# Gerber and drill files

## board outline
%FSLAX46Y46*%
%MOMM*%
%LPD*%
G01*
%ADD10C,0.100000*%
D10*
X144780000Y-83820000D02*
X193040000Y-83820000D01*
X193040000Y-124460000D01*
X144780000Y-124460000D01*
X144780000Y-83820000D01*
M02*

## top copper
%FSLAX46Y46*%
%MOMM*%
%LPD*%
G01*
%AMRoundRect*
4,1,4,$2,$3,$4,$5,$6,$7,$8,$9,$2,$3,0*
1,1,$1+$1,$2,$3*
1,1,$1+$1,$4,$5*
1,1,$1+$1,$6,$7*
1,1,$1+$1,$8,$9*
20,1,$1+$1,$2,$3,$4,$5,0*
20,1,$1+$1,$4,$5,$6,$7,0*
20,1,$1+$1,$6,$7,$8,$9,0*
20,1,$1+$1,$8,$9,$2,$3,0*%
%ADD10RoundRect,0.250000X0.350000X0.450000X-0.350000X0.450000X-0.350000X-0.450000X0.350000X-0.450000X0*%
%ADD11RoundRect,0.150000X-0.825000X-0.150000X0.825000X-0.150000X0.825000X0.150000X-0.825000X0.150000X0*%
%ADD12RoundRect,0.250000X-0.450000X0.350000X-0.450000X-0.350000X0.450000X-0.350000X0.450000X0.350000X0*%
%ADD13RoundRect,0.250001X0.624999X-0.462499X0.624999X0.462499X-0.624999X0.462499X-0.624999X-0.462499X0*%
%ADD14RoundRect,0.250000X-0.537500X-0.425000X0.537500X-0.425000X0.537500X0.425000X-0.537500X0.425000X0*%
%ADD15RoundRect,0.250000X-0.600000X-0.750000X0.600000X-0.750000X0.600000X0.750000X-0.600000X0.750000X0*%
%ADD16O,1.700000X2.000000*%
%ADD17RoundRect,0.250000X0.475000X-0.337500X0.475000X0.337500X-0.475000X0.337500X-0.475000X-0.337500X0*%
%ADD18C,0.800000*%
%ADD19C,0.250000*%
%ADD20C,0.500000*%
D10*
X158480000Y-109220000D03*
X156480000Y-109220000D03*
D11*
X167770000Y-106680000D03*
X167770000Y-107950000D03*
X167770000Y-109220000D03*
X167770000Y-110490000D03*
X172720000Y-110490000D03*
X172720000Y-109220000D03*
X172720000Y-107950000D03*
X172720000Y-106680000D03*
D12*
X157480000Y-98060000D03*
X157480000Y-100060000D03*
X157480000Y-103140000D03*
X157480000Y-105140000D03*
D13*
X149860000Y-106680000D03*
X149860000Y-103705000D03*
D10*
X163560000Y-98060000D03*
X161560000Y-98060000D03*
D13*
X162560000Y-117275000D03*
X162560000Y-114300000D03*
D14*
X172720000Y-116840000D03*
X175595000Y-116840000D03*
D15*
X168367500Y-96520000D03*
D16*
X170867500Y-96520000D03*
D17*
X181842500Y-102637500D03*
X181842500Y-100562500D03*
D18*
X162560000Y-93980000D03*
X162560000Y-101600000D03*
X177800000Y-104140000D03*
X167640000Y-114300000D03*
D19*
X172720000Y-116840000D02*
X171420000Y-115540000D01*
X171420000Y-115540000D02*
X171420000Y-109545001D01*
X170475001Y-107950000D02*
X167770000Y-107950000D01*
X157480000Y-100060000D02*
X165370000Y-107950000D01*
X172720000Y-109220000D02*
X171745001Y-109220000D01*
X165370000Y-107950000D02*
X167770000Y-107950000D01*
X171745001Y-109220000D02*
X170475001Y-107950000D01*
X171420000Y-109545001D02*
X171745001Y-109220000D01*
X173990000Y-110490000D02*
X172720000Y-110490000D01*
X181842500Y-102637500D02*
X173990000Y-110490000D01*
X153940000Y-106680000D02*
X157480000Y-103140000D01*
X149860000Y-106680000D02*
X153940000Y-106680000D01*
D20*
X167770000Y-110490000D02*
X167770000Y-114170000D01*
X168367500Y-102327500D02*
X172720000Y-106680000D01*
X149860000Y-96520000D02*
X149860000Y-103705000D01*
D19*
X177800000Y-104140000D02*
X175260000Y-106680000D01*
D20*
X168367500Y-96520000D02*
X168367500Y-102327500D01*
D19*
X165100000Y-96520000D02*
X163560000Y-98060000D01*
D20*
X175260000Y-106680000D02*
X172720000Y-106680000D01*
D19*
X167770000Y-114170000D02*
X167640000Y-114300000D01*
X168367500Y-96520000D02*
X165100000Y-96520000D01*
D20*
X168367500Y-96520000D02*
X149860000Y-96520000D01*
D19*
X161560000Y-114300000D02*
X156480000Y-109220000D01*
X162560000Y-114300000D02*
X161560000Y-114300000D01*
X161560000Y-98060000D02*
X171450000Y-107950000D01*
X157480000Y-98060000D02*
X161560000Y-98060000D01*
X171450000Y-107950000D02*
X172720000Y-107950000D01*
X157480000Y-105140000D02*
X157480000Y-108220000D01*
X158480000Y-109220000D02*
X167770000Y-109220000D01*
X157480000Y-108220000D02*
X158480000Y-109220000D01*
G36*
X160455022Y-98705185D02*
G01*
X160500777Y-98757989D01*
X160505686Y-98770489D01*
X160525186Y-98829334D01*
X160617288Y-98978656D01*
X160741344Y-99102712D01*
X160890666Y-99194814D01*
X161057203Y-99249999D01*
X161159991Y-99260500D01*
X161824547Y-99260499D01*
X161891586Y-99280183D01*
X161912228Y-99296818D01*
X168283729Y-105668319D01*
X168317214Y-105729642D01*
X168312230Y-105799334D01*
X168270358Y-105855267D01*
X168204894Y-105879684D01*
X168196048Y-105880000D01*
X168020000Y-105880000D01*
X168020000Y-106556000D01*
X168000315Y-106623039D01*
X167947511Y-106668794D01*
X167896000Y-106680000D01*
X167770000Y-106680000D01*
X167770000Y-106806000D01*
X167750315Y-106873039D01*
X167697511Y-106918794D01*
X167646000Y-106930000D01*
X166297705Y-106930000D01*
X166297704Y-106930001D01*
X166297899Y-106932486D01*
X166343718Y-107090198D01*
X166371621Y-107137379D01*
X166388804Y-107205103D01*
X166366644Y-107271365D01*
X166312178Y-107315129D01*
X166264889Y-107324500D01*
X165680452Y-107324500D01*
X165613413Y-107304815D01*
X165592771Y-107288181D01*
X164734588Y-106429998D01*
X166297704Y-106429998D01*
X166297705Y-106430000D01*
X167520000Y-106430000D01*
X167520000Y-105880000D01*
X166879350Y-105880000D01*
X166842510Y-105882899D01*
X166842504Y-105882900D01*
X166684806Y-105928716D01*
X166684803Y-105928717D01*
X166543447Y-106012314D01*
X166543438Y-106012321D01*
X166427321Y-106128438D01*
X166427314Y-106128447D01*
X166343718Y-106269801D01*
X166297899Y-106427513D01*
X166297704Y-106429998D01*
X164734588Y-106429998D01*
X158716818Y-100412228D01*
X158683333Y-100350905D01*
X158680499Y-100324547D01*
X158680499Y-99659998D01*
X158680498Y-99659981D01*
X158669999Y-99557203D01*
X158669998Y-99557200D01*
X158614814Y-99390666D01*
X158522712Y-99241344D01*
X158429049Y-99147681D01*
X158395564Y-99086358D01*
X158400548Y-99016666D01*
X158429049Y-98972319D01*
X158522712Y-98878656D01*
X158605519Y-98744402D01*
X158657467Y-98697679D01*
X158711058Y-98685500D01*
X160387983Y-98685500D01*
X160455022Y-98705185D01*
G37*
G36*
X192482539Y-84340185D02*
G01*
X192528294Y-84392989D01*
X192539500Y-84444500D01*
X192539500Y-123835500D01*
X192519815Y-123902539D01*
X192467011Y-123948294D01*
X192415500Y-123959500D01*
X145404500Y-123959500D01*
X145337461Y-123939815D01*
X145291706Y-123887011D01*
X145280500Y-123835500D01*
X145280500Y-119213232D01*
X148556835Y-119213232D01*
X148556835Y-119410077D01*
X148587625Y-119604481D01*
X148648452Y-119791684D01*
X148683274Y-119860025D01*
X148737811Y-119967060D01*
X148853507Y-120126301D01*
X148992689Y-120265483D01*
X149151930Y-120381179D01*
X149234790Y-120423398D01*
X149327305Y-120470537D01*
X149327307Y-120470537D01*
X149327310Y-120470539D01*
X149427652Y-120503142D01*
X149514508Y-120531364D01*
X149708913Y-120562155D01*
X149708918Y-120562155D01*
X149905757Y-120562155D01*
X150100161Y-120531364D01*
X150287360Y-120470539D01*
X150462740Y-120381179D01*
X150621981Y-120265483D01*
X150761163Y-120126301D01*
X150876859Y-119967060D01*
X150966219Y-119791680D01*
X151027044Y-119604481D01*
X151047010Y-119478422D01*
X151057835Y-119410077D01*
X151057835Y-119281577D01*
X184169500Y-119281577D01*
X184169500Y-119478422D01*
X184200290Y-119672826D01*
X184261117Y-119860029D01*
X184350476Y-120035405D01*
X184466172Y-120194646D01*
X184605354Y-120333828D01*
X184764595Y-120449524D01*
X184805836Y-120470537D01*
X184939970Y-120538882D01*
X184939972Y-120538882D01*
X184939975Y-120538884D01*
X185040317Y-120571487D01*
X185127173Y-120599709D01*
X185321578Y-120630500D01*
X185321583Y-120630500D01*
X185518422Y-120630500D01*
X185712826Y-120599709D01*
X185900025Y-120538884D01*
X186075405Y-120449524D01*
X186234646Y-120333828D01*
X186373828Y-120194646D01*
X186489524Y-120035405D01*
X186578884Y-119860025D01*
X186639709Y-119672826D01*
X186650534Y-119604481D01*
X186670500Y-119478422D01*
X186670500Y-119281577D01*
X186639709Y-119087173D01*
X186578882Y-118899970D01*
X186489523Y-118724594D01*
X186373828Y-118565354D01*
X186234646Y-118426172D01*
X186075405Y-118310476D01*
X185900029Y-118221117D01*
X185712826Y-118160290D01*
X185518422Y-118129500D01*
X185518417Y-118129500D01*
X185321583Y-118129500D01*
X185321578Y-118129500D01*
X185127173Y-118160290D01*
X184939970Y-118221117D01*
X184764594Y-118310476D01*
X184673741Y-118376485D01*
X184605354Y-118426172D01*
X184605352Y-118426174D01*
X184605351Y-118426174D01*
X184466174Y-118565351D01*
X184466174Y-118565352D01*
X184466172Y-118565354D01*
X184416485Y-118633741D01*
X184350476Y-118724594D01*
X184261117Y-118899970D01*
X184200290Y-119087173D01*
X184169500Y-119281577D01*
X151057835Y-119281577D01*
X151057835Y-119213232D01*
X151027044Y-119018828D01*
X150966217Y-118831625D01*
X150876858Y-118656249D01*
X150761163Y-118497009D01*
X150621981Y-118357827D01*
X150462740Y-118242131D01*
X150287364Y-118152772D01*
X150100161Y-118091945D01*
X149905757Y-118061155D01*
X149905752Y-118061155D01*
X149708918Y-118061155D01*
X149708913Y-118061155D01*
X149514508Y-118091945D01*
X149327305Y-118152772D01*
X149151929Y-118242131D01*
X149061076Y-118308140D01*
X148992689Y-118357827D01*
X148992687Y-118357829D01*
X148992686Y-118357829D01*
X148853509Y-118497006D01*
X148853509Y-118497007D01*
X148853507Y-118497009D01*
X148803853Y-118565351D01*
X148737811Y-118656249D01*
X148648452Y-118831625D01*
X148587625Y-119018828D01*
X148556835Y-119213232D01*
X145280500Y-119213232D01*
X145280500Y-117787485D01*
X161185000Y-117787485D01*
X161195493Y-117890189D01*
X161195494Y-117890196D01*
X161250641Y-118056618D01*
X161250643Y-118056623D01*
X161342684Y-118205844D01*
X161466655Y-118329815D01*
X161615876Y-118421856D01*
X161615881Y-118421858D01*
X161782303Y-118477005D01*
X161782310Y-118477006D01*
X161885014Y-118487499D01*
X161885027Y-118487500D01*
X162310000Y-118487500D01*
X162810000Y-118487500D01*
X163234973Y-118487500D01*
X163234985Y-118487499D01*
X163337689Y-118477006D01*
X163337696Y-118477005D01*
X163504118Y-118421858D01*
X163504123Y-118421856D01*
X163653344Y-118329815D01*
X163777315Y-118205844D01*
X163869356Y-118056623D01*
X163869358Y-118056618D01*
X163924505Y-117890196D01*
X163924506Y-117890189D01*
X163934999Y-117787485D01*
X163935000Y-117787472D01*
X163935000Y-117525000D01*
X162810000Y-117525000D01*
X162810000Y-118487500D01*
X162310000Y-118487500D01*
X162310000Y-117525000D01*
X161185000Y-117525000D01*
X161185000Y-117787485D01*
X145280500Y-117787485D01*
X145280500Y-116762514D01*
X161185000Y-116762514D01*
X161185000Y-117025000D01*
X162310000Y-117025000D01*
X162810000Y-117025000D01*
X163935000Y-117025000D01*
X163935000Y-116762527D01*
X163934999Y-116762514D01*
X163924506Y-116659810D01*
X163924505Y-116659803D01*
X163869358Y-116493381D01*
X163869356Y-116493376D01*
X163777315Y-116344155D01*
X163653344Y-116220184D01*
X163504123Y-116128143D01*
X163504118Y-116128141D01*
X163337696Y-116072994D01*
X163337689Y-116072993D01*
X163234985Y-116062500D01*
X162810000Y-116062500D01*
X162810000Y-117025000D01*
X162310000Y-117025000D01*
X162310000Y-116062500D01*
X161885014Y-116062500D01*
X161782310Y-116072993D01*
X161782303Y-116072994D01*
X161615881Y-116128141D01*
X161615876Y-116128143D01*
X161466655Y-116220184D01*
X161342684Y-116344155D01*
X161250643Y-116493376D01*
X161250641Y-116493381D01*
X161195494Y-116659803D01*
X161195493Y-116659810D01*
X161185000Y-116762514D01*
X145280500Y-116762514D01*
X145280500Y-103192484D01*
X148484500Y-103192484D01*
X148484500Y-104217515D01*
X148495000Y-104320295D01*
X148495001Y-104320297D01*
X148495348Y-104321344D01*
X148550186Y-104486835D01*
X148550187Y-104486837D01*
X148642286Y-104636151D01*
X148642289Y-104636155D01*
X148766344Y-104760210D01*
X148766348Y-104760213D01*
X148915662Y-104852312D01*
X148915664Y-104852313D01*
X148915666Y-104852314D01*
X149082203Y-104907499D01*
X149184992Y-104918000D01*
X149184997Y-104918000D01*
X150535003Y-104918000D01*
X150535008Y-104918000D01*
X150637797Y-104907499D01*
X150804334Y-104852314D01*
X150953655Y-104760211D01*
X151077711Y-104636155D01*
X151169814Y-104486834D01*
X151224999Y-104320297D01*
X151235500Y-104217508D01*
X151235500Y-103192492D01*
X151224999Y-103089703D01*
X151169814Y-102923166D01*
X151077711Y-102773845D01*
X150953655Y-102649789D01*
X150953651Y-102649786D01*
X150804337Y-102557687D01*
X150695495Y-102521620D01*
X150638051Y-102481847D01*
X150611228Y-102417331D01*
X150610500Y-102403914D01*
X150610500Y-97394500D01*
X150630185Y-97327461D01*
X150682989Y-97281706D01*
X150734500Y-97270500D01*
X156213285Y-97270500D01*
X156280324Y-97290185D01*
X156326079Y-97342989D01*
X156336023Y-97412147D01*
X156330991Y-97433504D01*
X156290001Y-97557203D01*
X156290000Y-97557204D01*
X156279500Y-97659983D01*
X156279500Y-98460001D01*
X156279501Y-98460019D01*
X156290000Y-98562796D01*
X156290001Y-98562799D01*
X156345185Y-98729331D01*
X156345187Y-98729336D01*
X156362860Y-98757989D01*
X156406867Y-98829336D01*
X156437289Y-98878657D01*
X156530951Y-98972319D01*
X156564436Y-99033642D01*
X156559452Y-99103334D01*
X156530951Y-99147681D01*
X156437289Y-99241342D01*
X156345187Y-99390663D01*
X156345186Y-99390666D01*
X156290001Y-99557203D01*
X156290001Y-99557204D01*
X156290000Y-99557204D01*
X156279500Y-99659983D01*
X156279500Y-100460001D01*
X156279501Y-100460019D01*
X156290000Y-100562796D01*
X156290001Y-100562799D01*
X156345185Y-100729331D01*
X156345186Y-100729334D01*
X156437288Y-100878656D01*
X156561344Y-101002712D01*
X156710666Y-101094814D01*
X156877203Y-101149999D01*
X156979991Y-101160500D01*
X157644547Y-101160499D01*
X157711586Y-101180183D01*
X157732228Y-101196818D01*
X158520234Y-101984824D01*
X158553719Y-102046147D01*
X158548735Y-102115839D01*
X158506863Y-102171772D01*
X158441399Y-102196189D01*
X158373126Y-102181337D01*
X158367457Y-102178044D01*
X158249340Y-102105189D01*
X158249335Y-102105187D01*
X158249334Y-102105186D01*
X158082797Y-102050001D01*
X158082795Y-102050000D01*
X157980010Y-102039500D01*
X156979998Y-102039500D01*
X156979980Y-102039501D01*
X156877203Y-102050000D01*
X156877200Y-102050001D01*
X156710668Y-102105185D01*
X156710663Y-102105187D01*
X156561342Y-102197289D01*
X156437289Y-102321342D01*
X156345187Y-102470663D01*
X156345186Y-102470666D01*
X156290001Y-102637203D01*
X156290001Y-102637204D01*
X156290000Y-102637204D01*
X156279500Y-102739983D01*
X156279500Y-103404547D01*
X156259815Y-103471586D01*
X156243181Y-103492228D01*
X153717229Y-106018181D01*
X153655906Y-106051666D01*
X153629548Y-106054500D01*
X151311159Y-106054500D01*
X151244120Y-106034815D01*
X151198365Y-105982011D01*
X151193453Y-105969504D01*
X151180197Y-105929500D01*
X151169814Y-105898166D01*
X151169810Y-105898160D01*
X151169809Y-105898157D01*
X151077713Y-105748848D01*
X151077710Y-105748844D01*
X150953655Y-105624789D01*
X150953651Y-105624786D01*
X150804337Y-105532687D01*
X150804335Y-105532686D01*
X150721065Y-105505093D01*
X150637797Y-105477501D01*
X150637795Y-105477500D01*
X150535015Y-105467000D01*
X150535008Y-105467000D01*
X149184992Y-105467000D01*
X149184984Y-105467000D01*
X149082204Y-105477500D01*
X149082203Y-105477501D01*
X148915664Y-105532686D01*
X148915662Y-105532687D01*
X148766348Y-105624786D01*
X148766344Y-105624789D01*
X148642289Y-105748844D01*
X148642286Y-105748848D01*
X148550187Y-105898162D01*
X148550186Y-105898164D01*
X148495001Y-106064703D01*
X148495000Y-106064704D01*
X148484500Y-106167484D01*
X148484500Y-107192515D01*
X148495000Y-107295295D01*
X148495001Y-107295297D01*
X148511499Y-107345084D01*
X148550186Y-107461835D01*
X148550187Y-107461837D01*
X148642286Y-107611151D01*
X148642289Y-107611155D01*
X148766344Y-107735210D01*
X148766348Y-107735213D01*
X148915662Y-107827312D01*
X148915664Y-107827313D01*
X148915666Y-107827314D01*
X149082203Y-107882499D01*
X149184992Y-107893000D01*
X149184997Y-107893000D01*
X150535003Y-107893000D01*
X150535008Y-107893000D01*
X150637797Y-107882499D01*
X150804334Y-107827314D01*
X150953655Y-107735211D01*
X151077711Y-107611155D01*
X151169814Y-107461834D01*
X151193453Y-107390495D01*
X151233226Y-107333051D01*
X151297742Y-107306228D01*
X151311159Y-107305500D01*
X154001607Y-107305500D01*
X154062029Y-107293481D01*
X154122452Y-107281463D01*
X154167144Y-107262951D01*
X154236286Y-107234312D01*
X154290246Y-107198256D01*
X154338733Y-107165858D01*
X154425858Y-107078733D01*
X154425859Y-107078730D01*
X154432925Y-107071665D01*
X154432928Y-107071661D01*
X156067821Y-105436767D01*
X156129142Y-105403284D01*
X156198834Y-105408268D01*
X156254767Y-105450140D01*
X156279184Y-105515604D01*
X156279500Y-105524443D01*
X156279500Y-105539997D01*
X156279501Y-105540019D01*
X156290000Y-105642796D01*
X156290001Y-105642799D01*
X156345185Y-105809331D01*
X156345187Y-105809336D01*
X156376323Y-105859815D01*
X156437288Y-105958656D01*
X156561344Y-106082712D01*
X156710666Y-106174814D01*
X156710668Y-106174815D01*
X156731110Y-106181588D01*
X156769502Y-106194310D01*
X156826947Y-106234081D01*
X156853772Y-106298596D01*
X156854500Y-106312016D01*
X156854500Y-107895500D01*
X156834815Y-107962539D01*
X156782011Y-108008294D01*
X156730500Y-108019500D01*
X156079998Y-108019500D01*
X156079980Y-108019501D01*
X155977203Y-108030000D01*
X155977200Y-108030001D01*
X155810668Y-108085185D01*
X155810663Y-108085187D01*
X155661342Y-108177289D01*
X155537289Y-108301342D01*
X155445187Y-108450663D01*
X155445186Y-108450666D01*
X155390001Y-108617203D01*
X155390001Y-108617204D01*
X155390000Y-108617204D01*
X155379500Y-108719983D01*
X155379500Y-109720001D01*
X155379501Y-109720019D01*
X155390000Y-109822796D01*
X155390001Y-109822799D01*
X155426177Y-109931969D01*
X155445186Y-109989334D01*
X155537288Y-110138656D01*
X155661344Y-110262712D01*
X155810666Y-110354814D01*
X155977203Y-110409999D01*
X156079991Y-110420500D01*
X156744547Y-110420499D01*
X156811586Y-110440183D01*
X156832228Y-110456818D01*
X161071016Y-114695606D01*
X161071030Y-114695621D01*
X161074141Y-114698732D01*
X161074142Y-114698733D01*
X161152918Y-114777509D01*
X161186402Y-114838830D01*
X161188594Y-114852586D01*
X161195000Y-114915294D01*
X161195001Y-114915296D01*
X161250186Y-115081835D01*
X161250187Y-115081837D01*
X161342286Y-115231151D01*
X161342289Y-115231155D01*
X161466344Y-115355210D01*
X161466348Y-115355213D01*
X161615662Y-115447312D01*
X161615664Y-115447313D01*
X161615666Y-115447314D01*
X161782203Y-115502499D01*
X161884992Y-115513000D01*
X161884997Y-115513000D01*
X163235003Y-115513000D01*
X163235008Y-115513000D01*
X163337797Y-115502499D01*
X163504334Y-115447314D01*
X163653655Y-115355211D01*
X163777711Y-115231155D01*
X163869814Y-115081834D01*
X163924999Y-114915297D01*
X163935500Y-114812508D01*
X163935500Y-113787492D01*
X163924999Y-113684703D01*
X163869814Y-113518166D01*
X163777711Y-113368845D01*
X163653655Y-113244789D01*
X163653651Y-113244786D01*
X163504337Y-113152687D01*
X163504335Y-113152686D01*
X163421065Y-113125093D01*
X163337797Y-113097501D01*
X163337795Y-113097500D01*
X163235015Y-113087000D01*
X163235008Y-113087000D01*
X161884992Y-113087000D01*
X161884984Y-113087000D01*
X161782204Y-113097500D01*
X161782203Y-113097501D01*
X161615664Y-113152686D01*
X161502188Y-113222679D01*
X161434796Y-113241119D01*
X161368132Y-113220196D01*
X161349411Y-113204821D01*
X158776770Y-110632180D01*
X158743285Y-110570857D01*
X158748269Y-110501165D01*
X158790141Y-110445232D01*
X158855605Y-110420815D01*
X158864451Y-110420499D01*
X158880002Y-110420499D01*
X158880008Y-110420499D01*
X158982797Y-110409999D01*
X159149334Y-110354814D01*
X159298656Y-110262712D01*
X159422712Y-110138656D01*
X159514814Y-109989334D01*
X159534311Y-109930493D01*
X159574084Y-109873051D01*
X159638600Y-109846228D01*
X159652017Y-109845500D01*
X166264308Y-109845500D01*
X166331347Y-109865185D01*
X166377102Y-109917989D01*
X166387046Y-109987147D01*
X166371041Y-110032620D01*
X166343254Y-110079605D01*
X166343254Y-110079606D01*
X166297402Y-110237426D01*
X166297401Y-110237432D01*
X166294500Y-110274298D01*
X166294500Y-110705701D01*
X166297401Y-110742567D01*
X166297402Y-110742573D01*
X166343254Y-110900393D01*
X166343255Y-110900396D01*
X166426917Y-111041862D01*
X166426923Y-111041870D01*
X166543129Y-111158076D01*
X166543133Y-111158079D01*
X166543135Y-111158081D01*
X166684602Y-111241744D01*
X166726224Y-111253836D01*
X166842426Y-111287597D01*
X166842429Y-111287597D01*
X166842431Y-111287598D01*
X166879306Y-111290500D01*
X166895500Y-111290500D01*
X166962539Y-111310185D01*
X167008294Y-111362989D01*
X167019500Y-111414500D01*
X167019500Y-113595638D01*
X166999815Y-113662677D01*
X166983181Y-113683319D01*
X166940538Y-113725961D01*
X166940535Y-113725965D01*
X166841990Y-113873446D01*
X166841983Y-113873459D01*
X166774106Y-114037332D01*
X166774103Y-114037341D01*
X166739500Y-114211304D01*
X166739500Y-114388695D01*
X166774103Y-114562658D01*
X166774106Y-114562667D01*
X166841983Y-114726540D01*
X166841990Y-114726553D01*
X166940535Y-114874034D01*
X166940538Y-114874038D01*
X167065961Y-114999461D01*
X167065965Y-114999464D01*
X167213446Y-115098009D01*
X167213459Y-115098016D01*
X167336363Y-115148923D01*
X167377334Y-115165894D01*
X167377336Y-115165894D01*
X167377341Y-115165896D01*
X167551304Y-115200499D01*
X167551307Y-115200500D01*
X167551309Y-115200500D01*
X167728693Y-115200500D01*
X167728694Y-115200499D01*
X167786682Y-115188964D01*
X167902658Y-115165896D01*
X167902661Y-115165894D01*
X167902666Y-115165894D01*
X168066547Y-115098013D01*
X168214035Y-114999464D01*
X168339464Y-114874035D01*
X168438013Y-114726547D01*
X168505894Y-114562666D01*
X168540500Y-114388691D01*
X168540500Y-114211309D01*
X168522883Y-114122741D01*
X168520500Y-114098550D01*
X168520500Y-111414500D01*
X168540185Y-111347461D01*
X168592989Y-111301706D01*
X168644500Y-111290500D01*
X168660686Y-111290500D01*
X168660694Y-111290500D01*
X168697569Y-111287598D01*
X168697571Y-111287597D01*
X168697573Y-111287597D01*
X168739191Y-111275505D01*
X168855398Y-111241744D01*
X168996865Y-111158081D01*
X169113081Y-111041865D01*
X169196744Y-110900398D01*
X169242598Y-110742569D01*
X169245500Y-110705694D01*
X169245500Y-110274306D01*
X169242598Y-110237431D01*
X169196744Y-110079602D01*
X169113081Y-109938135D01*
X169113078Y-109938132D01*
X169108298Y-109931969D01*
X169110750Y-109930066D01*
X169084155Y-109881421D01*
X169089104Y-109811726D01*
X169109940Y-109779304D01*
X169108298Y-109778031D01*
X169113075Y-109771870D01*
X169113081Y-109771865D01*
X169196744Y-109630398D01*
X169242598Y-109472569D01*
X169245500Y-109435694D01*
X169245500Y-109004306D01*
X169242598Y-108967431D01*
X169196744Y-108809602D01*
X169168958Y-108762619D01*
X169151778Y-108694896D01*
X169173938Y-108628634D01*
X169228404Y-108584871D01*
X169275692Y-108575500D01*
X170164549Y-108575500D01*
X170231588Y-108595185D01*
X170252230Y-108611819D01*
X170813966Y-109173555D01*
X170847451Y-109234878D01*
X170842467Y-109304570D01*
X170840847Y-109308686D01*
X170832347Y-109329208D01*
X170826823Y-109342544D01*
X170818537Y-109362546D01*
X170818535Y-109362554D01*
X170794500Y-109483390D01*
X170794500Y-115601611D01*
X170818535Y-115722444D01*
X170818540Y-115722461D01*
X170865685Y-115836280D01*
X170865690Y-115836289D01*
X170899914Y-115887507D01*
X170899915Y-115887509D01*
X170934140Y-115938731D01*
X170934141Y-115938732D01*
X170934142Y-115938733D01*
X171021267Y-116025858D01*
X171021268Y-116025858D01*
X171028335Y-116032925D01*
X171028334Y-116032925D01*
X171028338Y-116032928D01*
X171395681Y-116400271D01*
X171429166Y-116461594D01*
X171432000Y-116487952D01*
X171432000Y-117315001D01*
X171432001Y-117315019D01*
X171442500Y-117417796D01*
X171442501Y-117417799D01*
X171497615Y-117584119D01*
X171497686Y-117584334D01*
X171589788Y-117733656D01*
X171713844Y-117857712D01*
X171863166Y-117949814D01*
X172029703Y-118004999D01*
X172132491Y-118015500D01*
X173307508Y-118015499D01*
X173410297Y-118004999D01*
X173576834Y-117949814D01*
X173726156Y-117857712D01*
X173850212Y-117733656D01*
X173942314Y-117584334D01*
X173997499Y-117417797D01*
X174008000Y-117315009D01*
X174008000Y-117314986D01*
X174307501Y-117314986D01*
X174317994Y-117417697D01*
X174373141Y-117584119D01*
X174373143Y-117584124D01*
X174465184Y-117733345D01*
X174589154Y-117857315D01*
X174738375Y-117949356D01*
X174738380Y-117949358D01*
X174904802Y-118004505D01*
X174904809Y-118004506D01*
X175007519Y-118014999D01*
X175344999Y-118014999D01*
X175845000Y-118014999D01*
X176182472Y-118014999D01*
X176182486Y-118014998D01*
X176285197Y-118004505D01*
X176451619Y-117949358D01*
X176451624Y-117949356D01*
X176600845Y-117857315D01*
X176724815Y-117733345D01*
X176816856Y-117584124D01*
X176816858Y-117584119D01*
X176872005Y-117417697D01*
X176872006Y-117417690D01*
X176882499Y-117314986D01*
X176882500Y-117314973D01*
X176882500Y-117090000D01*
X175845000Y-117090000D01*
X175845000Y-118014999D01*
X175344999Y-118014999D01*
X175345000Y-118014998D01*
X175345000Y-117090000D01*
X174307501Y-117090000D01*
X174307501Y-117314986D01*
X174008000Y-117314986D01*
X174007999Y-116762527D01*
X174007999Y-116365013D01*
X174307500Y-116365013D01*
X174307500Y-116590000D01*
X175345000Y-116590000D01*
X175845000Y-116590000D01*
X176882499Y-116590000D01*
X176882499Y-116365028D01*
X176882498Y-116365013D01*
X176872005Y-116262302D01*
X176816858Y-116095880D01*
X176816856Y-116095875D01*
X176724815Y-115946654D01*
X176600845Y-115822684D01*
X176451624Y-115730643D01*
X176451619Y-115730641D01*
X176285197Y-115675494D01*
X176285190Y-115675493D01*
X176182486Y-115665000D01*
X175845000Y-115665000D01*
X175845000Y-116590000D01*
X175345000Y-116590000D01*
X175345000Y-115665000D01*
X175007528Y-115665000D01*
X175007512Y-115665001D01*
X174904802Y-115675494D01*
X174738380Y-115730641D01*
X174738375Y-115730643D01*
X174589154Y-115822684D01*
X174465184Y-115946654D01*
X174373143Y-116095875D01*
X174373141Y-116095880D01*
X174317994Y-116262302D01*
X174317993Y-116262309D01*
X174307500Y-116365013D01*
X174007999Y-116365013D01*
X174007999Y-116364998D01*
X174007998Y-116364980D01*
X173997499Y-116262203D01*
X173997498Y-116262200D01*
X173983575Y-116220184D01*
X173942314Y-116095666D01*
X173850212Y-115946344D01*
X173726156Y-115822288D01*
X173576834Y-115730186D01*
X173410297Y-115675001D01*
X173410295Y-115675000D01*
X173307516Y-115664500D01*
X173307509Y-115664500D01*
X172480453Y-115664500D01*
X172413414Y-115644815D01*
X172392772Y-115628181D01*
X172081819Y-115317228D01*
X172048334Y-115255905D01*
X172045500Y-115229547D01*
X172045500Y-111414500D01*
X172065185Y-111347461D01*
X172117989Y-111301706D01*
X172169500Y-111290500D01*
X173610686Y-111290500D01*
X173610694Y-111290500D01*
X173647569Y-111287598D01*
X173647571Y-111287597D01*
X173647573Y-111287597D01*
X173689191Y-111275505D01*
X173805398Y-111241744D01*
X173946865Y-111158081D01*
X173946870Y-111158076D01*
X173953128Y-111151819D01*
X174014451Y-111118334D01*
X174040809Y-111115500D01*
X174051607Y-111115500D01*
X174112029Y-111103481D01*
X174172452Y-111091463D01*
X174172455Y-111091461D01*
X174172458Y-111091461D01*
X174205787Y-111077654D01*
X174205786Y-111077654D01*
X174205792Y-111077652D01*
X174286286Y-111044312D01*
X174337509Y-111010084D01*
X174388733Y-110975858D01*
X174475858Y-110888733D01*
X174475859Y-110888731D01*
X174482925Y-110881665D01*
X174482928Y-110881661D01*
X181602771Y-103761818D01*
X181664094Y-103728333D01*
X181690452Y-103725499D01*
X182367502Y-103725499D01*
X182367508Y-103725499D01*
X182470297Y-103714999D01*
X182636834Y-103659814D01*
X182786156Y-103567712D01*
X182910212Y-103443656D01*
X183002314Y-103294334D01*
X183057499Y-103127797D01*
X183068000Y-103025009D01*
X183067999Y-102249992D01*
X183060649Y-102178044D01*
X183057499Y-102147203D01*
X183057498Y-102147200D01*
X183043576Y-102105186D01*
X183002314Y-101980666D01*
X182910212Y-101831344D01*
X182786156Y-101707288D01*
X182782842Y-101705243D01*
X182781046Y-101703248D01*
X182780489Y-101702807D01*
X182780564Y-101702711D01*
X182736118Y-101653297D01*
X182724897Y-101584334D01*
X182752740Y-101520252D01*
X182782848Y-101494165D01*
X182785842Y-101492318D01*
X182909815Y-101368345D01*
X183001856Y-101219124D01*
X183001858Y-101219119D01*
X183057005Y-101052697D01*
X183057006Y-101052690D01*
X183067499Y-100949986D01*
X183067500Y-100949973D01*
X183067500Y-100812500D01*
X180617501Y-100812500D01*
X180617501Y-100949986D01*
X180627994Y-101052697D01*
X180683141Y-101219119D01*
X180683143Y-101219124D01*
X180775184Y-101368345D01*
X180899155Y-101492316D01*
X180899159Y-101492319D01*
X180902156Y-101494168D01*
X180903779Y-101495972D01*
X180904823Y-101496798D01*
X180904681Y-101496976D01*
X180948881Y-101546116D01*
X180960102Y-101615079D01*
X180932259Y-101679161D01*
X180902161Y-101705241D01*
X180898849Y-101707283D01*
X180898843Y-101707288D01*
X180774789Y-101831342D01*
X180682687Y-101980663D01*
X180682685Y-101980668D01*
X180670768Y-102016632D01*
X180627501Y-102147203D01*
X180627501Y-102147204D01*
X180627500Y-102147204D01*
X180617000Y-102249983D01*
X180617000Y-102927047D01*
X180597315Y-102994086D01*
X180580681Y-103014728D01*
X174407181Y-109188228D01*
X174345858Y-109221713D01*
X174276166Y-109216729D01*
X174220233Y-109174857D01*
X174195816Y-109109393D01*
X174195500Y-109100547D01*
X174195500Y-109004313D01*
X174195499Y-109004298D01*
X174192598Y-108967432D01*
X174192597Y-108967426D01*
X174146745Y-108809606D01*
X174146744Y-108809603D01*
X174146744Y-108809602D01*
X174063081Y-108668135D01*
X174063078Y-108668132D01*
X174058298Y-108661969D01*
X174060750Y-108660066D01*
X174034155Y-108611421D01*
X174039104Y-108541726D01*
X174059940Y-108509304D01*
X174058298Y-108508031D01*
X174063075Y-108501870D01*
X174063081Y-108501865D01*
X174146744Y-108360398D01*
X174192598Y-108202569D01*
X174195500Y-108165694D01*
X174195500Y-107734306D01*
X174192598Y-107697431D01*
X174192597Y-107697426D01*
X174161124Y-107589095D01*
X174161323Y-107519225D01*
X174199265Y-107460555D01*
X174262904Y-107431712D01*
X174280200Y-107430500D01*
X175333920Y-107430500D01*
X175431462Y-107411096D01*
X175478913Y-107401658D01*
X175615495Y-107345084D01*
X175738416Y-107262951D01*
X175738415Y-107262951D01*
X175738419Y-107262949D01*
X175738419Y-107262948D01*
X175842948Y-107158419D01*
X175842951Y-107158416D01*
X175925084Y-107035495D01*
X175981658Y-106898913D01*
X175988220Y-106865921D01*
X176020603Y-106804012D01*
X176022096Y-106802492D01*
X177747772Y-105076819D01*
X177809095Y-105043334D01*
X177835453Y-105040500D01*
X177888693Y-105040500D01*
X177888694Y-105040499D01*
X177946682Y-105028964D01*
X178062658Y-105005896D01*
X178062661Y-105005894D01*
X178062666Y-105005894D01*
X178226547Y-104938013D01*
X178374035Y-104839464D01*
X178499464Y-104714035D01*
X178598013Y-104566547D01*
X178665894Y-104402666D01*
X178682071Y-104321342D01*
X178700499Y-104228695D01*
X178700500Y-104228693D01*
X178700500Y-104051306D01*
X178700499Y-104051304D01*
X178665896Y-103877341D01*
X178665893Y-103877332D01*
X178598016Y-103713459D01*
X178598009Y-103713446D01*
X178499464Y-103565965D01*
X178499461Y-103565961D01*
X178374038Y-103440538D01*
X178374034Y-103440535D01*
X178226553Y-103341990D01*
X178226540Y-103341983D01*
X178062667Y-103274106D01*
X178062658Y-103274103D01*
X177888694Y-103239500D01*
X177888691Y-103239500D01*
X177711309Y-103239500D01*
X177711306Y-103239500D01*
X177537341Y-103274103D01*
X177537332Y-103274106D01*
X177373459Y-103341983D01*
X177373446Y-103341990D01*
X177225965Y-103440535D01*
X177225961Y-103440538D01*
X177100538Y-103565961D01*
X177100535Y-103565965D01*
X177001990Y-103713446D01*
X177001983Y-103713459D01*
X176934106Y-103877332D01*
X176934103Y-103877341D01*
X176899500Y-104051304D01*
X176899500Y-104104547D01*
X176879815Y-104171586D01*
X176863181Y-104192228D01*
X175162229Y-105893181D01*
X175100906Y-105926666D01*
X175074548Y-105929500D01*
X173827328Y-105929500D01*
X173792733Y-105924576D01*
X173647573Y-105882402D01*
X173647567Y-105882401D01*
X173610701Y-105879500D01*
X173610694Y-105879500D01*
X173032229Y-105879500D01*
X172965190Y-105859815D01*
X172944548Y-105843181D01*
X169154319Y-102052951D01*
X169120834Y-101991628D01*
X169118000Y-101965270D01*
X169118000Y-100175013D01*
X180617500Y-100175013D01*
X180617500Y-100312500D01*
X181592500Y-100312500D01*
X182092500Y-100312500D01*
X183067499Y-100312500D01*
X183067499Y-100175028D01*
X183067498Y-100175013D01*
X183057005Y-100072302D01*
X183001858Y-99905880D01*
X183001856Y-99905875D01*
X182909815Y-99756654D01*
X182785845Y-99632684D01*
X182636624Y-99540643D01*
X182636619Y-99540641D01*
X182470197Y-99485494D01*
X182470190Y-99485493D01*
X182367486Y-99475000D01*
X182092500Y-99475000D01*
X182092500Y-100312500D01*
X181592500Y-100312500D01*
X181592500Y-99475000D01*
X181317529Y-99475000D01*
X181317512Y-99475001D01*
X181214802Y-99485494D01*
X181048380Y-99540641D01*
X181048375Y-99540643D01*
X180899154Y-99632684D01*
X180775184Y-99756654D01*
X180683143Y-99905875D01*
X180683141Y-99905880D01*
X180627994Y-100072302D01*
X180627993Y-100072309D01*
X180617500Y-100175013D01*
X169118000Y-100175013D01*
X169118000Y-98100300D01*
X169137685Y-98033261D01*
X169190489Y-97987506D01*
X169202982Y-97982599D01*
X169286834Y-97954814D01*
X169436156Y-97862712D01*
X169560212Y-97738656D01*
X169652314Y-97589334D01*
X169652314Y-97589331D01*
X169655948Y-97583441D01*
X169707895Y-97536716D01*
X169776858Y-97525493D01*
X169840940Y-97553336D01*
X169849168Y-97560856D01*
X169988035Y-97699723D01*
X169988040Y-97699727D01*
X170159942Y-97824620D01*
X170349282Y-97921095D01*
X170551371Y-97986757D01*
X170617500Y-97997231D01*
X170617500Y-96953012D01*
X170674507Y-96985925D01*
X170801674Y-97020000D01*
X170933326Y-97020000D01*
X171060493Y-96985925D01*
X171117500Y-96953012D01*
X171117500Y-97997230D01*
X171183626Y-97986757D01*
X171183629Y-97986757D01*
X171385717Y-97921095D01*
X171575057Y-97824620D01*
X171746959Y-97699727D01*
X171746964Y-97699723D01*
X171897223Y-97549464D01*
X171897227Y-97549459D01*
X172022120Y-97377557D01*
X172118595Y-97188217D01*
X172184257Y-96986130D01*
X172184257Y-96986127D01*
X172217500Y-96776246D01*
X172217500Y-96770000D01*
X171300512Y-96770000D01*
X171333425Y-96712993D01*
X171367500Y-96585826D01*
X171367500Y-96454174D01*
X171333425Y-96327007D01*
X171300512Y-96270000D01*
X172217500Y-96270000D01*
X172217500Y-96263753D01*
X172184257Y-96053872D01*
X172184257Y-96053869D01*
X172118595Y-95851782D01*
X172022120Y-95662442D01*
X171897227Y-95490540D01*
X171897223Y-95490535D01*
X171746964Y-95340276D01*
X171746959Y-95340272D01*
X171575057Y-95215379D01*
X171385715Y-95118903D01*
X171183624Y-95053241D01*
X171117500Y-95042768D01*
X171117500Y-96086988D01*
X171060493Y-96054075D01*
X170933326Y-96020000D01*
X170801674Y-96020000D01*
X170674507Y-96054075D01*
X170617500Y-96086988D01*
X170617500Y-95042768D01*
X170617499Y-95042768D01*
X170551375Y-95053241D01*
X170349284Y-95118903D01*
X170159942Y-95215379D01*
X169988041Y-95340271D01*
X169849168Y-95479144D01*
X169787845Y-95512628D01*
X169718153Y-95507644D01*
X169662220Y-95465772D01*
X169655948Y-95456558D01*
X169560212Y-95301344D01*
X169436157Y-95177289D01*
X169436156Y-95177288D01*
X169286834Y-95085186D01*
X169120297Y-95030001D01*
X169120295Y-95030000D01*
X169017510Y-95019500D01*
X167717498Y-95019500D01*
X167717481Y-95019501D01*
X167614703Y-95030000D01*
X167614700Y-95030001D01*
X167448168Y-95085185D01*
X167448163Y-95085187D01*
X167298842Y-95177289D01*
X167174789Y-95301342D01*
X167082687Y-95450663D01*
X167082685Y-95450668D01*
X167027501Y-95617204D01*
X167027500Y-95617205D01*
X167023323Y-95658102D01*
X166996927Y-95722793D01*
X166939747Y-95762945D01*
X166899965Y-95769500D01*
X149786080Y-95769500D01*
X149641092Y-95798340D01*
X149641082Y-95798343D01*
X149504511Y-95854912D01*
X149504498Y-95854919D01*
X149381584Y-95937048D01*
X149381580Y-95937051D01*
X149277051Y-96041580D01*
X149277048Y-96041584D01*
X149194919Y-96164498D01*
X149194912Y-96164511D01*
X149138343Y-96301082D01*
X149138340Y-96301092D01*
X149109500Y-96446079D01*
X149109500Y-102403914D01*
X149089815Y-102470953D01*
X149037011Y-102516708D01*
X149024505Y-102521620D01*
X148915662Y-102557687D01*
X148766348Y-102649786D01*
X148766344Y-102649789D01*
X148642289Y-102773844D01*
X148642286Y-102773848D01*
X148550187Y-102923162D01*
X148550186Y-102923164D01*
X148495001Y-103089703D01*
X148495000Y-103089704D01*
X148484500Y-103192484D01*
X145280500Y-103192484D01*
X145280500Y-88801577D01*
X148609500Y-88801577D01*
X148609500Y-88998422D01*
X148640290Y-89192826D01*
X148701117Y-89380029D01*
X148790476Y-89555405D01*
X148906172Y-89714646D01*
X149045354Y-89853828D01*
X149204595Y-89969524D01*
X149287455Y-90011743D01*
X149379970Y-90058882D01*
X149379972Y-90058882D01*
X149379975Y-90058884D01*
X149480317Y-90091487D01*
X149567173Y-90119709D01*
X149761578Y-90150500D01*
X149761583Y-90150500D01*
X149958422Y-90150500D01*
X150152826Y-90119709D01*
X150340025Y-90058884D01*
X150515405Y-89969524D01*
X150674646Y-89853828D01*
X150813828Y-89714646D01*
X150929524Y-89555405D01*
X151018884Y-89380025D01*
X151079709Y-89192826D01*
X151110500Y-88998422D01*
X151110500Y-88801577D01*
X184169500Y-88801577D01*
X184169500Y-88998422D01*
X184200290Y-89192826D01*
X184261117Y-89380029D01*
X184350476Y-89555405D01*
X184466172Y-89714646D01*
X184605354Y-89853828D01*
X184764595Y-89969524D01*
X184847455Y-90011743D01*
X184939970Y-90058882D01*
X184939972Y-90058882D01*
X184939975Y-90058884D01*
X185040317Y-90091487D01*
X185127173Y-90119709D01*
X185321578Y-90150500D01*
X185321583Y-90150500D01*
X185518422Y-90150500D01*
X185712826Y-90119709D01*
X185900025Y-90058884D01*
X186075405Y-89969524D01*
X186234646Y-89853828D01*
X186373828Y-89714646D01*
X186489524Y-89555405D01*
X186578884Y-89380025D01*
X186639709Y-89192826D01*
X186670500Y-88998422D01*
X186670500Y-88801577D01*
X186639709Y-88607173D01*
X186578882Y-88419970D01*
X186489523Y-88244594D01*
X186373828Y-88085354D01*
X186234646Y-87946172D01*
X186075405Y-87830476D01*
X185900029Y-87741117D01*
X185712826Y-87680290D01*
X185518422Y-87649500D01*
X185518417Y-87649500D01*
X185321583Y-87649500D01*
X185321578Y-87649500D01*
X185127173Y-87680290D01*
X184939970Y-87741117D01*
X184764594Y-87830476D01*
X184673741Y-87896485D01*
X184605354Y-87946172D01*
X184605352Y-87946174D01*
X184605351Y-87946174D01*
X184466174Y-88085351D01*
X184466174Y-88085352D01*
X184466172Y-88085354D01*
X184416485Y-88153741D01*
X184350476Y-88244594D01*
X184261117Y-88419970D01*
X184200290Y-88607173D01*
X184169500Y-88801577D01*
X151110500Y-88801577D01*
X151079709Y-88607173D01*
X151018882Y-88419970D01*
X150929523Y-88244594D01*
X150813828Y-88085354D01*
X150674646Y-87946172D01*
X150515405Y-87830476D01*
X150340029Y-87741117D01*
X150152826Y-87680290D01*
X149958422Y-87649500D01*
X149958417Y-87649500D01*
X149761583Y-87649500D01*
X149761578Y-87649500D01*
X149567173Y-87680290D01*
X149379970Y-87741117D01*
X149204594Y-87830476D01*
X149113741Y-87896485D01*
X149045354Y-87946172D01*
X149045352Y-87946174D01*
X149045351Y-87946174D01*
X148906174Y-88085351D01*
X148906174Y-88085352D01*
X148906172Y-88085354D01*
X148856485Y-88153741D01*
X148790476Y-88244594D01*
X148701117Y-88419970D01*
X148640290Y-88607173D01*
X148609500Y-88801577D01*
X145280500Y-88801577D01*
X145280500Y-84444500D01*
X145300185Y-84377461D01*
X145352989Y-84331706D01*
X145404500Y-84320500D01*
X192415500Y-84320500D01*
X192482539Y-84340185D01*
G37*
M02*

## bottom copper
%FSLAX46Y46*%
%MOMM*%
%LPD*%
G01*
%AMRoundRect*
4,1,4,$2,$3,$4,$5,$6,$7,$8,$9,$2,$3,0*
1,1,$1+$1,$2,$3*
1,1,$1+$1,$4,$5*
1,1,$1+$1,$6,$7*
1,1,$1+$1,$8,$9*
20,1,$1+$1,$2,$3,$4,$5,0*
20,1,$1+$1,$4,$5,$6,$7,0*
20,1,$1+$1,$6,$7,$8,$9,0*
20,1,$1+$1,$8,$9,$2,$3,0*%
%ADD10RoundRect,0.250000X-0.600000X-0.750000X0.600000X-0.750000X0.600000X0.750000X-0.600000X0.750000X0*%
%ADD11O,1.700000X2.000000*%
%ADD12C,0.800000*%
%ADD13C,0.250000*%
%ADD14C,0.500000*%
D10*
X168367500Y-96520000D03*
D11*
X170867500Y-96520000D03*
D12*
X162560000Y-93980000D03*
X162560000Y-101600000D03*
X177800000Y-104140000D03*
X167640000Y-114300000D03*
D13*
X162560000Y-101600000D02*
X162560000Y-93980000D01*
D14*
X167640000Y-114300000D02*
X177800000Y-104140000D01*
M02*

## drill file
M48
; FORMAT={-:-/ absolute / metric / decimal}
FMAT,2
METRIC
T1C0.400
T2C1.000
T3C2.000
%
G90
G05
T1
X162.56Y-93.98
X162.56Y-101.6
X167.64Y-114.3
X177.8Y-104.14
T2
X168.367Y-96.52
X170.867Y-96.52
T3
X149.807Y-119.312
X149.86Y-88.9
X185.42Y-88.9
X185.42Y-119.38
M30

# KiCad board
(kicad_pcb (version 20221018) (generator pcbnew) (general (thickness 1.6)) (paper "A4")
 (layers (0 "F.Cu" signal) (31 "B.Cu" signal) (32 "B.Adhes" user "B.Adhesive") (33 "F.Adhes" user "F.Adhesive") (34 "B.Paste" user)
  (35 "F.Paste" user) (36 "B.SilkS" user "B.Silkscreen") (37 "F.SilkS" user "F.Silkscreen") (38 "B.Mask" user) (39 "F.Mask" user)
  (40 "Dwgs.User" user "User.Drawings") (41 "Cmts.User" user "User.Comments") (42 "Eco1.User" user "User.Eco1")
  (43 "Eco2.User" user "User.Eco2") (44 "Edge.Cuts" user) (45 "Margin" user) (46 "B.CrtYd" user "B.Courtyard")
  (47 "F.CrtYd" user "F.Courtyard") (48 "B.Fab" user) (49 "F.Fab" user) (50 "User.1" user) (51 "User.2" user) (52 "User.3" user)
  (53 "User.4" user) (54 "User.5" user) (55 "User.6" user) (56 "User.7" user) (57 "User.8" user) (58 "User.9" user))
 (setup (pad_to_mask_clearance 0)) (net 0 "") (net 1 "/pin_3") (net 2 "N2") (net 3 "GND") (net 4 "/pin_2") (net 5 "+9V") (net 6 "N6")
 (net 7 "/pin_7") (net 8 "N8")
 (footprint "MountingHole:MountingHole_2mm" (layer "F.Cu") (at 185.42 119.38)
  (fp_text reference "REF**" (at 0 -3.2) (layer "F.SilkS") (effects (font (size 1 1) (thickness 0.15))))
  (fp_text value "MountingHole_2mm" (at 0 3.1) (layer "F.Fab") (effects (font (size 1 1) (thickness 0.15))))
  (pad "" np_thru_hole circle (at 0 0) (size 2 2) (drill 2) (layers "F&B.Cu" "*.Mask")))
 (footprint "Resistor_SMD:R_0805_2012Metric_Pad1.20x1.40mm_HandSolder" (layer "F.Cu") (at 157.48 109.22 180)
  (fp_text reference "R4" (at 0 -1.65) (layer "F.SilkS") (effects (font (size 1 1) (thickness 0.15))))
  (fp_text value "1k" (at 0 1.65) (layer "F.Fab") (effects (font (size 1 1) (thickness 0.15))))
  (pad "1" smd roundrect (at -1 0 180) (size 1.2 1.4) (layers "F.Cu" "F.Paste" "F.Mask") (roundrect_rratio 0.2083333333) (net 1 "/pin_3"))
  (pad "2" smd roundrect (at 1 0 180) (size 1.2 1.4) (layers "F.Cu" "F.Paste" "F.Mask") (roundrect_rratio 0.2083333333) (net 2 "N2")))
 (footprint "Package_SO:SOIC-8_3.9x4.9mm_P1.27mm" (layer "F.Cu") (at 170.245 108.585)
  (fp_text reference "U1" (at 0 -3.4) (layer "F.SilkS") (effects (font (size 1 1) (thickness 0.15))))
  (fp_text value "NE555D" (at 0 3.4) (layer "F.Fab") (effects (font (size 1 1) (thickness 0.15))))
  (pad "1" smd roundrect (at -2.475 -1.905) (size 1.95 0.6) (layers "F.Cu" "F.Paste" "F.Mask") (roundrect_rratio 0.25) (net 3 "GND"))
  (pad "2" smd roundrect (at -2.475 -0.635) (size 1.95 0.6) (layers "F.Cu" "F.Paste" "F.Mask") (roundrect_rratio 0.25) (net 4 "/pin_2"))
  (pad "3" smd roundrect (at -2.475 0.635) (size 1.95 0.6) (layers "F.Cu" "F.Paste" "F.Mask") (roundrect_rratio 0.25) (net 1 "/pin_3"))
  (pad "4" smd roundrect (at -2.475 1.905) (size 1.95 0.6) (layers "F.Cu" "F.Paste" "F.Mask") (roundrect_rratio 0.25) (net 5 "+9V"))
  (pad "5" smd roundrect (at 2.475 1.905) (size 1.95 0.6) (layers "F.Cu" "F.Paste" "F.Mask") (roundrect_rratio 0.25) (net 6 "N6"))
  (pad "6" smd roundrect (at 2.475 0.635) (size 1.95 0.6) (layers "F.Cu" "F.Paste" "F.Mask") (roundrect_rratio 0.25) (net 4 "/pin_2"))
  (pad "7" smd roundrect (at 2.475 -0.635) (size 1.95 0.6) (layers "F.Cu" "F.Paste" "F.Mask") (roundrect_rratio 0.25) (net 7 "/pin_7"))
  (pad "8" smd roundrect (at 2.475 -1.905) (size 1.95 0.6) (layers "F.Cu" "F.Paste" "F.Mask") (roundrect_rratio 0.25) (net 5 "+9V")))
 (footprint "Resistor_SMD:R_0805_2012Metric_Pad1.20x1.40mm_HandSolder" (layer "F.Cu") (at 157.48 99.06 -90)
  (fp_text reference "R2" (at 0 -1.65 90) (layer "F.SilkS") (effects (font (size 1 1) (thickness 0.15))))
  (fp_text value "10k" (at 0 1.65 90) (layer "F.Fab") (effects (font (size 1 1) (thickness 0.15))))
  (pad "1" smd roundrect (at -1 0 270) (size 1.2 1.4) (layers "F.Cu" "F.Paste" "F.Mask") (roundrect_rratio 0.2083333333) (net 7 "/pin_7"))
  (pad "2" smd roundrect (at 1 0 270) (size 1.2 1.4) (layers "F.Cu" "F.Paste" "F.Mask") (roundrect_rratio 0.2083333333) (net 4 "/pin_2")))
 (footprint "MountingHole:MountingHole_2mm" (layer "F.Cu") (at 149.807335 119.311655)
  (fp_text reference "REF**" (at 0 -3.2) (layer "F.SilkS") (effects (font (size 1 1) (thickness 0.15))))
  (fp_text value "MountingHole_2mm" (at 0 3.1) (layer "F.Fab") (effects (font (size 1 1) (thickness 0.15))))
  (pad "" np_thru_hole circle (at 0 0) (size 2 2) (drill 2) (layers "F&B.Cu" "*.Mask")))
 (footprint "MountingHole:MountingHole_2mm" (layer "F.Cu") (at 149.86 88.9)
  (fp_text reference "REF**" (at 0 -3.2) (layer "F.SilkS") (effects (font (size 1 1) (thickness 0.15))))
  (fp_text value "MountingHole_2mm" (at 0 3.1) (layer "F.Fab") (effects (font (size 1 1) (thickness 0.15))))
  (pad "" np_thru_hole circle (at 0 0) (size 2 2) (drill 2) (layers "F&B.Cu" "*.Mask")))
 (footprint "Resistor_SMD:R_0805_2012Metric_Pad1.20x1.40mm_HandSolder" (layer "F.Cu") (at 157.48 104.14 -90)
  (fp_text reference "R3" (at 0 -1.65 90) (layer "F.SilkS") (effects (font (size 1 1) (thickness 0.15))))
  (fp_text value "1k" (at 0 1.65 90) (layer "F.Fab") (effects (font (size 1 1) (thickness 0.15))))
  (pad "1" smd roundrect (at -1 0 270) (size 1.2 1.4) (layers "F.Cu" "F.Paste" "F.Mask") (roundrect_rratio 0.2083333333) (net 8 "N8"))
  (pad "2" smd roundrect (at 1 0 270) (size 1.2 1.4) (layers "F.Cu" "F.Paste" "F.Mask") (roundrect_rratio 0.2083333333) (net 1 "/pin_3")))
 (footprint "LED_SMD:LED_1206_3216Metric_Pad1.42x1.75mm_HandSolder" (layer "F.Cu") (at 149.86 105.1925 90)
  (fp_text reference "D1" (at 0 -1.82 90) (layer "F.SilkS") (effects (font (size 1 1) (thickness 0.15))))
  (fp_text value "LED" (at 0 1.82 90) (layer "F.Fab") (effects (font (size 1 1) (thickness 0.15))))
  (pad "1" smd roundrect (at -1.4875 0 90) (size 1.425 1.75) (layers "F.Cu" "F.Paste" "F.Mask") (roundrect_rratio 0.1754392982) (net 8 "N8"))
  (pad "2" smd roundrect (at 1.4875 0 90) (size 1.425 1.75) (layers "F.Cu" "F.Paste" "F.Mask") (roundrect_rratio 0.1754392982) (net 5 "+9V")))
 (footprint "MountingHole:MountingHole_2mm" (layer "F.Cu") (at 185.42 88.9)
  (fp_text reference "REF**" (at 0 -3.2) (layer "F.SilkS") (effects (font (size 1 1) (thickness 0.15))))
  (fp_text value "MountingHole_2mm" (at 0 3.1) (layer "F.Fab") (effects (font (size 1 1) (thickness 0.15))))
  (pad "" np_thru_hole circle (at 0 0) (size 2 2) (drill 2) (layers "*.Cu" "*.Mask")))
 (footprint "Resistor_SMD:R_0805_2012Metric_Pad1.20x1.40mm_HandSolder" (layer "F.Cu") (at 162.56 98.06 180)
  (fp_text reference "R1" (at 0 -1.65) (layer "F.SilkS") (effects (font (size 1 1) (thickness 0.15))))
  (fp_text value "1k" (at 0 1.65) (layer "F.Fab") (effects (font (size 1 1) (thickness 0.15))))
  (pad "1" smd roundrect (at -1 0 180) (size 1.2 1.4) (layers "F.Cu" "F.Paste" "F.Mask") (roundrect_rratio 0.2083333333) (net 5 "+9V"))
  (pad "2" smd roundrect (at 1 0 180) (size 1.2 1.4) (layers "F.Cu" "F.Paste" "F.Mask") (roundrect_rratio 0.2083333333) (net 7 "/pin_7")))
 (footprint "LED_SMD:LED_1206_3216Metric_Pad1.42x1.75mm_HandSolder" (layer "F.Cu") (at 162.56 115.7875 90)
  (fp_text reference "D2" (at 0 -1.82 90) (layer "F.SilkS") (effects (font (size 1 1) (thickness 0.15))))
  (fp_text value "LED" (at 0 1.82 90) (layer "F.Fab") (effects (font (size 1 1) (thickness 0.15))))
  (pad "1" smd roundrect (at -1.4875 0 90) (size 1.425 1.75) (layers "F.Cu" "F.Paste" "F.Mask") (roundrect_rratio 0.1754392982)
   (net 3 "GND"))
  (pad "2" smd roundrect (at 1.4875 0 90) (size 1.425 1.75) (layers "F.Cu" "F.Paste" "F.Mask") (roundrect_rratio 0.1754392982) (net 2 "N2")))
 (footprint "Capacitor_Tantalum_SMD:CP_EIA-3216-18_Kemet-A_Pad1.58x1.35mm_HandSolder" (layer "F.Cu") (at 174.1575 116.84)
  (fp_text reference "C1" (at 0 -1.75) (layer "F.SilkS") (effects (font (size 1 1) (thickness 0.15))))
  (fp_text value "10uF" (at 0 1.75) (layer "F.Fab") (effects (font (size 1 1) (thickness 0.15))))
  (pad "1" smd roundrect (at -1.4375 0) (size 1.575 1.35) (layers "F.Cu" "F.Paste" "F.Mask") (roundrect_rratio 0.1851851852)
   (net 4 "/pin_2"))
  (pad "2" smd roundrect (at 1.4375 0) (size 1.575 1.35) (layers "F.Cu" "F.Paste" "F.Mask") (roundrect_rratio 0.1851851852) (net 3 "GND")))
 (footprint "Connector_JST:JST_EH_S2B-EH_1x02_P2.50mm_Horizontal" (layer "F.Cu") (at 168.3675 96.52)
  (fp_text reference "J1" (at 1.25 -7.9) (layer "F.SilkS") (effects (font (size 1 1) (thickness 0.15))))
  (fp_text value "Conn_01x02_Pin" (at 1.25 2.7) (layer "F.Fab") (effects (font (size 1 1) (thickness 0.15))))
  (pad "1" thru_hole roundrect (at 0 0) (size 1.7 2) (drill 1) (layers "*.Cu" "*.Mask") (roundrect_rratio 0.1470588235) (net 5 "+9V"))
  (pad "2" thru_hole oval (at 2.5 0) (size 1.7 2) (drill 1) (layers "*.Cu" "*.Mask") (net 3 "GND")))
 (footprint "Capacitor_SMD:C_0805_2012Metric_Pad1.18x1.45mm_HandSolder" (layer "F.Cu") (at 181.8425 101.6 90)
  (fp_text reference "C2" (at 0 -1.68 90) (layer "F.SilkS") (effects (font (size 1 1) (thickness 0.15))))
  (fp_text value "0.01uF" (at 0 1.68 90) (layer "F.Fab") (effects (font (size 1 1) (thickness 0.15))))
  (pad "1" smd roundrect (at -1.0375 0 90) (size 1.175 1.45) (layers "F.Cu" "F.Paste" "F.Mask") (roundrect_rratio 0.2127659574) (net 6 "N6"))
  (pad "2" smd roundrect (at 1.0375 0 90) (size 1.175 1.45) (layers "F.Cu" "F.Paste" "F.Mask") (roundrect_rratio 0.2127659574) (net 3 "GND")))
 (gr_rect (start 144.78 83.82) (end 193.04 124.46) (stroke (width 0.1) (type default)) (fill none) (layer "Edge.Cuts"))
 (segment (start 172.72 116.84) (end 171.42 115.54) (width 0.25) (layer "F.Cu") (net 4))
 (segment (start 171.42 115.54) (end 171.42 109.545001) (width 0.25) (layer "F.Cu") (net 4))
 (segment (start 170.475001 107.95) (end 167.77 107.95) (width 0.25) (layer "F.Cu") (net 4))
 (segment (start 157.48 100.06) (end 165.37 107.95) (width 0.25) (layer "F.Cu") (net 4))
 (segment (start 172.72 109.22) (end 171.745001 109.22) (width 0.25) (layer "F.Cu") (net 4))
 (segment (start 165.37 107.95) (end 167.77 107.95) (width 0.25) (layer "F.Cu") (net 4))
 (segment (start 171.745001 109.22) (end 170.475001 107.95) (width 0.25) (layer "F.Cu") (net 4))
 (segment (start 171.42 109.545001) (end 171.745001 109.22) (width 0.25) (layer "F.Cu") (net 4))
 (via (at 162.56 93.98) (size 0.8) (drill 0.4) (layers "F.Cu" "B.Cu") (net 3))
 (via (at 162.56 101.6) (size 0.8) (drill 0.4) (layers "F.Cu" "B.Cu") (free) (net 3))
 (segment (start 162.56 101.6) (end 162.56 93.98) (width 0.25) (layer "B.Cu") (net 3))
 (segment (start 173.99 110.49) (end 172.72 110.49) (width 0.25) (layer "F.Cu") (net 6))
 (segment (start 181.8425 102.6375) (end 173.99 110.49) (width 0.25) (layer "F.Cu") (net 6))
 (segment (start 153.94 106.68) (end 157.48 103.14) (width 0.25) (layer "F.Cu") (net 8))
 (segment (start 149.86 106.68) (end 153.94 106.68) (width 0.25) (layer "F.Cu") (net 8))
 (segment (start 167.77 110.49) (end 167.77 114.17) (width 0.5) (layer "F.Cu") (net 5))
 (segment (start 168.3675 102.3275) (end 172.72 106.68) (width 0.5) (layer "F.Cu") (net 5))
 (segment (start 149.86 96.52) (end 149.86 103.705) (width 0.5) (layer "F.Cu") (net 5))
 (segment (start 177.8 104.14) (end 175.26 106.68) (width 0.25) (layer "F.Cu") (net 5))
 (segment (start 168.3675 96.52) (end 168.3675 102.3275) (width 0.5) (layer "F.Cu") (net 5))
 (segment (start 165.1 96.52) (end 163.56 98.06) (width 0.25) (layer "F.Cu") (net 5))
 (segment (start 175.26 106.68) (end 172.72 106.68) (width 0.5) (layer "F.Cu") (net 5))
 (segment (start 167.77 114.17) (end 167.64 114.3) (width 0.25) (layer "F.Cu") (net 5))
 (segment (start 168.3675 96.52) (end 165.1 96.52) (width 0.25) (layer "F.Cu") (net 5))
 (segment (start 168.3675 96.52) (end 149.86 96.52) (width 0.5) (layer "F.Cu") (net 5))
 (via (at 177.8 104.14) (size 0.8) (drill 0.4) (layers "F.Cu" "B.Cu") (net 5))
 (via (at 167.64 114.3) (size 0.8) (drill 0.4) (layers "F.Cu" "B.Cu") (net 5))
 (segment (start 167.64 114.3) (end 177.8 104.14) (width 0.5) (layer "B.Cu") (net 5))
 (segment (start 161.56 114.3) (end 156.48 109.22) (width 0.25) (layer "F.Cu") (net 2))
 (segment (start 162.56 114.3) (end 161.56 114.3) (width 0.25) (layer "F.Cu") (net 2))
 (segment (start 161.56 98.06) (end 171.45 107.95) (width 0.25) (layer "F.Cu") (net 7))
 (segment (start 157.48 98.06) (end 161.56 98.06) (width 0.25) (layer "F.Cu") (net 7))
 (segment (start 171.45 107.95) (end 172.72 107.95) (width 0.25) (layer "F.Cu") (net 7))
 (segment (start 157.48 105.14) (end 157.48 108.22) (width 0.25) (layer "F.Cu") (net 1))
 (segment (start 158.48 109.22) (end 167.77 109.22) (width 0.25) (layer "F.Cu") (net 1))
 (segment (start 157.48 108.22) (end 158.48 109.22) (width 0.25) (layer "F.Cu") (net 1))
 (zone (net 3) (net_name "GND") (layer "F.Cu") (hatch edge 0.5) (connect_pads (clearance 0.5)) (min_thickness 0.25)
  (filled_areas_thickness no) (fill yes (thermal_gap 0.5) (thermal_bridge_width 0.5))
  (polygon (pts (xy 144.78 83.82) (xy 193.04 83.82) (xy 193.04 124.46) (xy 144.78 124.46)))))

